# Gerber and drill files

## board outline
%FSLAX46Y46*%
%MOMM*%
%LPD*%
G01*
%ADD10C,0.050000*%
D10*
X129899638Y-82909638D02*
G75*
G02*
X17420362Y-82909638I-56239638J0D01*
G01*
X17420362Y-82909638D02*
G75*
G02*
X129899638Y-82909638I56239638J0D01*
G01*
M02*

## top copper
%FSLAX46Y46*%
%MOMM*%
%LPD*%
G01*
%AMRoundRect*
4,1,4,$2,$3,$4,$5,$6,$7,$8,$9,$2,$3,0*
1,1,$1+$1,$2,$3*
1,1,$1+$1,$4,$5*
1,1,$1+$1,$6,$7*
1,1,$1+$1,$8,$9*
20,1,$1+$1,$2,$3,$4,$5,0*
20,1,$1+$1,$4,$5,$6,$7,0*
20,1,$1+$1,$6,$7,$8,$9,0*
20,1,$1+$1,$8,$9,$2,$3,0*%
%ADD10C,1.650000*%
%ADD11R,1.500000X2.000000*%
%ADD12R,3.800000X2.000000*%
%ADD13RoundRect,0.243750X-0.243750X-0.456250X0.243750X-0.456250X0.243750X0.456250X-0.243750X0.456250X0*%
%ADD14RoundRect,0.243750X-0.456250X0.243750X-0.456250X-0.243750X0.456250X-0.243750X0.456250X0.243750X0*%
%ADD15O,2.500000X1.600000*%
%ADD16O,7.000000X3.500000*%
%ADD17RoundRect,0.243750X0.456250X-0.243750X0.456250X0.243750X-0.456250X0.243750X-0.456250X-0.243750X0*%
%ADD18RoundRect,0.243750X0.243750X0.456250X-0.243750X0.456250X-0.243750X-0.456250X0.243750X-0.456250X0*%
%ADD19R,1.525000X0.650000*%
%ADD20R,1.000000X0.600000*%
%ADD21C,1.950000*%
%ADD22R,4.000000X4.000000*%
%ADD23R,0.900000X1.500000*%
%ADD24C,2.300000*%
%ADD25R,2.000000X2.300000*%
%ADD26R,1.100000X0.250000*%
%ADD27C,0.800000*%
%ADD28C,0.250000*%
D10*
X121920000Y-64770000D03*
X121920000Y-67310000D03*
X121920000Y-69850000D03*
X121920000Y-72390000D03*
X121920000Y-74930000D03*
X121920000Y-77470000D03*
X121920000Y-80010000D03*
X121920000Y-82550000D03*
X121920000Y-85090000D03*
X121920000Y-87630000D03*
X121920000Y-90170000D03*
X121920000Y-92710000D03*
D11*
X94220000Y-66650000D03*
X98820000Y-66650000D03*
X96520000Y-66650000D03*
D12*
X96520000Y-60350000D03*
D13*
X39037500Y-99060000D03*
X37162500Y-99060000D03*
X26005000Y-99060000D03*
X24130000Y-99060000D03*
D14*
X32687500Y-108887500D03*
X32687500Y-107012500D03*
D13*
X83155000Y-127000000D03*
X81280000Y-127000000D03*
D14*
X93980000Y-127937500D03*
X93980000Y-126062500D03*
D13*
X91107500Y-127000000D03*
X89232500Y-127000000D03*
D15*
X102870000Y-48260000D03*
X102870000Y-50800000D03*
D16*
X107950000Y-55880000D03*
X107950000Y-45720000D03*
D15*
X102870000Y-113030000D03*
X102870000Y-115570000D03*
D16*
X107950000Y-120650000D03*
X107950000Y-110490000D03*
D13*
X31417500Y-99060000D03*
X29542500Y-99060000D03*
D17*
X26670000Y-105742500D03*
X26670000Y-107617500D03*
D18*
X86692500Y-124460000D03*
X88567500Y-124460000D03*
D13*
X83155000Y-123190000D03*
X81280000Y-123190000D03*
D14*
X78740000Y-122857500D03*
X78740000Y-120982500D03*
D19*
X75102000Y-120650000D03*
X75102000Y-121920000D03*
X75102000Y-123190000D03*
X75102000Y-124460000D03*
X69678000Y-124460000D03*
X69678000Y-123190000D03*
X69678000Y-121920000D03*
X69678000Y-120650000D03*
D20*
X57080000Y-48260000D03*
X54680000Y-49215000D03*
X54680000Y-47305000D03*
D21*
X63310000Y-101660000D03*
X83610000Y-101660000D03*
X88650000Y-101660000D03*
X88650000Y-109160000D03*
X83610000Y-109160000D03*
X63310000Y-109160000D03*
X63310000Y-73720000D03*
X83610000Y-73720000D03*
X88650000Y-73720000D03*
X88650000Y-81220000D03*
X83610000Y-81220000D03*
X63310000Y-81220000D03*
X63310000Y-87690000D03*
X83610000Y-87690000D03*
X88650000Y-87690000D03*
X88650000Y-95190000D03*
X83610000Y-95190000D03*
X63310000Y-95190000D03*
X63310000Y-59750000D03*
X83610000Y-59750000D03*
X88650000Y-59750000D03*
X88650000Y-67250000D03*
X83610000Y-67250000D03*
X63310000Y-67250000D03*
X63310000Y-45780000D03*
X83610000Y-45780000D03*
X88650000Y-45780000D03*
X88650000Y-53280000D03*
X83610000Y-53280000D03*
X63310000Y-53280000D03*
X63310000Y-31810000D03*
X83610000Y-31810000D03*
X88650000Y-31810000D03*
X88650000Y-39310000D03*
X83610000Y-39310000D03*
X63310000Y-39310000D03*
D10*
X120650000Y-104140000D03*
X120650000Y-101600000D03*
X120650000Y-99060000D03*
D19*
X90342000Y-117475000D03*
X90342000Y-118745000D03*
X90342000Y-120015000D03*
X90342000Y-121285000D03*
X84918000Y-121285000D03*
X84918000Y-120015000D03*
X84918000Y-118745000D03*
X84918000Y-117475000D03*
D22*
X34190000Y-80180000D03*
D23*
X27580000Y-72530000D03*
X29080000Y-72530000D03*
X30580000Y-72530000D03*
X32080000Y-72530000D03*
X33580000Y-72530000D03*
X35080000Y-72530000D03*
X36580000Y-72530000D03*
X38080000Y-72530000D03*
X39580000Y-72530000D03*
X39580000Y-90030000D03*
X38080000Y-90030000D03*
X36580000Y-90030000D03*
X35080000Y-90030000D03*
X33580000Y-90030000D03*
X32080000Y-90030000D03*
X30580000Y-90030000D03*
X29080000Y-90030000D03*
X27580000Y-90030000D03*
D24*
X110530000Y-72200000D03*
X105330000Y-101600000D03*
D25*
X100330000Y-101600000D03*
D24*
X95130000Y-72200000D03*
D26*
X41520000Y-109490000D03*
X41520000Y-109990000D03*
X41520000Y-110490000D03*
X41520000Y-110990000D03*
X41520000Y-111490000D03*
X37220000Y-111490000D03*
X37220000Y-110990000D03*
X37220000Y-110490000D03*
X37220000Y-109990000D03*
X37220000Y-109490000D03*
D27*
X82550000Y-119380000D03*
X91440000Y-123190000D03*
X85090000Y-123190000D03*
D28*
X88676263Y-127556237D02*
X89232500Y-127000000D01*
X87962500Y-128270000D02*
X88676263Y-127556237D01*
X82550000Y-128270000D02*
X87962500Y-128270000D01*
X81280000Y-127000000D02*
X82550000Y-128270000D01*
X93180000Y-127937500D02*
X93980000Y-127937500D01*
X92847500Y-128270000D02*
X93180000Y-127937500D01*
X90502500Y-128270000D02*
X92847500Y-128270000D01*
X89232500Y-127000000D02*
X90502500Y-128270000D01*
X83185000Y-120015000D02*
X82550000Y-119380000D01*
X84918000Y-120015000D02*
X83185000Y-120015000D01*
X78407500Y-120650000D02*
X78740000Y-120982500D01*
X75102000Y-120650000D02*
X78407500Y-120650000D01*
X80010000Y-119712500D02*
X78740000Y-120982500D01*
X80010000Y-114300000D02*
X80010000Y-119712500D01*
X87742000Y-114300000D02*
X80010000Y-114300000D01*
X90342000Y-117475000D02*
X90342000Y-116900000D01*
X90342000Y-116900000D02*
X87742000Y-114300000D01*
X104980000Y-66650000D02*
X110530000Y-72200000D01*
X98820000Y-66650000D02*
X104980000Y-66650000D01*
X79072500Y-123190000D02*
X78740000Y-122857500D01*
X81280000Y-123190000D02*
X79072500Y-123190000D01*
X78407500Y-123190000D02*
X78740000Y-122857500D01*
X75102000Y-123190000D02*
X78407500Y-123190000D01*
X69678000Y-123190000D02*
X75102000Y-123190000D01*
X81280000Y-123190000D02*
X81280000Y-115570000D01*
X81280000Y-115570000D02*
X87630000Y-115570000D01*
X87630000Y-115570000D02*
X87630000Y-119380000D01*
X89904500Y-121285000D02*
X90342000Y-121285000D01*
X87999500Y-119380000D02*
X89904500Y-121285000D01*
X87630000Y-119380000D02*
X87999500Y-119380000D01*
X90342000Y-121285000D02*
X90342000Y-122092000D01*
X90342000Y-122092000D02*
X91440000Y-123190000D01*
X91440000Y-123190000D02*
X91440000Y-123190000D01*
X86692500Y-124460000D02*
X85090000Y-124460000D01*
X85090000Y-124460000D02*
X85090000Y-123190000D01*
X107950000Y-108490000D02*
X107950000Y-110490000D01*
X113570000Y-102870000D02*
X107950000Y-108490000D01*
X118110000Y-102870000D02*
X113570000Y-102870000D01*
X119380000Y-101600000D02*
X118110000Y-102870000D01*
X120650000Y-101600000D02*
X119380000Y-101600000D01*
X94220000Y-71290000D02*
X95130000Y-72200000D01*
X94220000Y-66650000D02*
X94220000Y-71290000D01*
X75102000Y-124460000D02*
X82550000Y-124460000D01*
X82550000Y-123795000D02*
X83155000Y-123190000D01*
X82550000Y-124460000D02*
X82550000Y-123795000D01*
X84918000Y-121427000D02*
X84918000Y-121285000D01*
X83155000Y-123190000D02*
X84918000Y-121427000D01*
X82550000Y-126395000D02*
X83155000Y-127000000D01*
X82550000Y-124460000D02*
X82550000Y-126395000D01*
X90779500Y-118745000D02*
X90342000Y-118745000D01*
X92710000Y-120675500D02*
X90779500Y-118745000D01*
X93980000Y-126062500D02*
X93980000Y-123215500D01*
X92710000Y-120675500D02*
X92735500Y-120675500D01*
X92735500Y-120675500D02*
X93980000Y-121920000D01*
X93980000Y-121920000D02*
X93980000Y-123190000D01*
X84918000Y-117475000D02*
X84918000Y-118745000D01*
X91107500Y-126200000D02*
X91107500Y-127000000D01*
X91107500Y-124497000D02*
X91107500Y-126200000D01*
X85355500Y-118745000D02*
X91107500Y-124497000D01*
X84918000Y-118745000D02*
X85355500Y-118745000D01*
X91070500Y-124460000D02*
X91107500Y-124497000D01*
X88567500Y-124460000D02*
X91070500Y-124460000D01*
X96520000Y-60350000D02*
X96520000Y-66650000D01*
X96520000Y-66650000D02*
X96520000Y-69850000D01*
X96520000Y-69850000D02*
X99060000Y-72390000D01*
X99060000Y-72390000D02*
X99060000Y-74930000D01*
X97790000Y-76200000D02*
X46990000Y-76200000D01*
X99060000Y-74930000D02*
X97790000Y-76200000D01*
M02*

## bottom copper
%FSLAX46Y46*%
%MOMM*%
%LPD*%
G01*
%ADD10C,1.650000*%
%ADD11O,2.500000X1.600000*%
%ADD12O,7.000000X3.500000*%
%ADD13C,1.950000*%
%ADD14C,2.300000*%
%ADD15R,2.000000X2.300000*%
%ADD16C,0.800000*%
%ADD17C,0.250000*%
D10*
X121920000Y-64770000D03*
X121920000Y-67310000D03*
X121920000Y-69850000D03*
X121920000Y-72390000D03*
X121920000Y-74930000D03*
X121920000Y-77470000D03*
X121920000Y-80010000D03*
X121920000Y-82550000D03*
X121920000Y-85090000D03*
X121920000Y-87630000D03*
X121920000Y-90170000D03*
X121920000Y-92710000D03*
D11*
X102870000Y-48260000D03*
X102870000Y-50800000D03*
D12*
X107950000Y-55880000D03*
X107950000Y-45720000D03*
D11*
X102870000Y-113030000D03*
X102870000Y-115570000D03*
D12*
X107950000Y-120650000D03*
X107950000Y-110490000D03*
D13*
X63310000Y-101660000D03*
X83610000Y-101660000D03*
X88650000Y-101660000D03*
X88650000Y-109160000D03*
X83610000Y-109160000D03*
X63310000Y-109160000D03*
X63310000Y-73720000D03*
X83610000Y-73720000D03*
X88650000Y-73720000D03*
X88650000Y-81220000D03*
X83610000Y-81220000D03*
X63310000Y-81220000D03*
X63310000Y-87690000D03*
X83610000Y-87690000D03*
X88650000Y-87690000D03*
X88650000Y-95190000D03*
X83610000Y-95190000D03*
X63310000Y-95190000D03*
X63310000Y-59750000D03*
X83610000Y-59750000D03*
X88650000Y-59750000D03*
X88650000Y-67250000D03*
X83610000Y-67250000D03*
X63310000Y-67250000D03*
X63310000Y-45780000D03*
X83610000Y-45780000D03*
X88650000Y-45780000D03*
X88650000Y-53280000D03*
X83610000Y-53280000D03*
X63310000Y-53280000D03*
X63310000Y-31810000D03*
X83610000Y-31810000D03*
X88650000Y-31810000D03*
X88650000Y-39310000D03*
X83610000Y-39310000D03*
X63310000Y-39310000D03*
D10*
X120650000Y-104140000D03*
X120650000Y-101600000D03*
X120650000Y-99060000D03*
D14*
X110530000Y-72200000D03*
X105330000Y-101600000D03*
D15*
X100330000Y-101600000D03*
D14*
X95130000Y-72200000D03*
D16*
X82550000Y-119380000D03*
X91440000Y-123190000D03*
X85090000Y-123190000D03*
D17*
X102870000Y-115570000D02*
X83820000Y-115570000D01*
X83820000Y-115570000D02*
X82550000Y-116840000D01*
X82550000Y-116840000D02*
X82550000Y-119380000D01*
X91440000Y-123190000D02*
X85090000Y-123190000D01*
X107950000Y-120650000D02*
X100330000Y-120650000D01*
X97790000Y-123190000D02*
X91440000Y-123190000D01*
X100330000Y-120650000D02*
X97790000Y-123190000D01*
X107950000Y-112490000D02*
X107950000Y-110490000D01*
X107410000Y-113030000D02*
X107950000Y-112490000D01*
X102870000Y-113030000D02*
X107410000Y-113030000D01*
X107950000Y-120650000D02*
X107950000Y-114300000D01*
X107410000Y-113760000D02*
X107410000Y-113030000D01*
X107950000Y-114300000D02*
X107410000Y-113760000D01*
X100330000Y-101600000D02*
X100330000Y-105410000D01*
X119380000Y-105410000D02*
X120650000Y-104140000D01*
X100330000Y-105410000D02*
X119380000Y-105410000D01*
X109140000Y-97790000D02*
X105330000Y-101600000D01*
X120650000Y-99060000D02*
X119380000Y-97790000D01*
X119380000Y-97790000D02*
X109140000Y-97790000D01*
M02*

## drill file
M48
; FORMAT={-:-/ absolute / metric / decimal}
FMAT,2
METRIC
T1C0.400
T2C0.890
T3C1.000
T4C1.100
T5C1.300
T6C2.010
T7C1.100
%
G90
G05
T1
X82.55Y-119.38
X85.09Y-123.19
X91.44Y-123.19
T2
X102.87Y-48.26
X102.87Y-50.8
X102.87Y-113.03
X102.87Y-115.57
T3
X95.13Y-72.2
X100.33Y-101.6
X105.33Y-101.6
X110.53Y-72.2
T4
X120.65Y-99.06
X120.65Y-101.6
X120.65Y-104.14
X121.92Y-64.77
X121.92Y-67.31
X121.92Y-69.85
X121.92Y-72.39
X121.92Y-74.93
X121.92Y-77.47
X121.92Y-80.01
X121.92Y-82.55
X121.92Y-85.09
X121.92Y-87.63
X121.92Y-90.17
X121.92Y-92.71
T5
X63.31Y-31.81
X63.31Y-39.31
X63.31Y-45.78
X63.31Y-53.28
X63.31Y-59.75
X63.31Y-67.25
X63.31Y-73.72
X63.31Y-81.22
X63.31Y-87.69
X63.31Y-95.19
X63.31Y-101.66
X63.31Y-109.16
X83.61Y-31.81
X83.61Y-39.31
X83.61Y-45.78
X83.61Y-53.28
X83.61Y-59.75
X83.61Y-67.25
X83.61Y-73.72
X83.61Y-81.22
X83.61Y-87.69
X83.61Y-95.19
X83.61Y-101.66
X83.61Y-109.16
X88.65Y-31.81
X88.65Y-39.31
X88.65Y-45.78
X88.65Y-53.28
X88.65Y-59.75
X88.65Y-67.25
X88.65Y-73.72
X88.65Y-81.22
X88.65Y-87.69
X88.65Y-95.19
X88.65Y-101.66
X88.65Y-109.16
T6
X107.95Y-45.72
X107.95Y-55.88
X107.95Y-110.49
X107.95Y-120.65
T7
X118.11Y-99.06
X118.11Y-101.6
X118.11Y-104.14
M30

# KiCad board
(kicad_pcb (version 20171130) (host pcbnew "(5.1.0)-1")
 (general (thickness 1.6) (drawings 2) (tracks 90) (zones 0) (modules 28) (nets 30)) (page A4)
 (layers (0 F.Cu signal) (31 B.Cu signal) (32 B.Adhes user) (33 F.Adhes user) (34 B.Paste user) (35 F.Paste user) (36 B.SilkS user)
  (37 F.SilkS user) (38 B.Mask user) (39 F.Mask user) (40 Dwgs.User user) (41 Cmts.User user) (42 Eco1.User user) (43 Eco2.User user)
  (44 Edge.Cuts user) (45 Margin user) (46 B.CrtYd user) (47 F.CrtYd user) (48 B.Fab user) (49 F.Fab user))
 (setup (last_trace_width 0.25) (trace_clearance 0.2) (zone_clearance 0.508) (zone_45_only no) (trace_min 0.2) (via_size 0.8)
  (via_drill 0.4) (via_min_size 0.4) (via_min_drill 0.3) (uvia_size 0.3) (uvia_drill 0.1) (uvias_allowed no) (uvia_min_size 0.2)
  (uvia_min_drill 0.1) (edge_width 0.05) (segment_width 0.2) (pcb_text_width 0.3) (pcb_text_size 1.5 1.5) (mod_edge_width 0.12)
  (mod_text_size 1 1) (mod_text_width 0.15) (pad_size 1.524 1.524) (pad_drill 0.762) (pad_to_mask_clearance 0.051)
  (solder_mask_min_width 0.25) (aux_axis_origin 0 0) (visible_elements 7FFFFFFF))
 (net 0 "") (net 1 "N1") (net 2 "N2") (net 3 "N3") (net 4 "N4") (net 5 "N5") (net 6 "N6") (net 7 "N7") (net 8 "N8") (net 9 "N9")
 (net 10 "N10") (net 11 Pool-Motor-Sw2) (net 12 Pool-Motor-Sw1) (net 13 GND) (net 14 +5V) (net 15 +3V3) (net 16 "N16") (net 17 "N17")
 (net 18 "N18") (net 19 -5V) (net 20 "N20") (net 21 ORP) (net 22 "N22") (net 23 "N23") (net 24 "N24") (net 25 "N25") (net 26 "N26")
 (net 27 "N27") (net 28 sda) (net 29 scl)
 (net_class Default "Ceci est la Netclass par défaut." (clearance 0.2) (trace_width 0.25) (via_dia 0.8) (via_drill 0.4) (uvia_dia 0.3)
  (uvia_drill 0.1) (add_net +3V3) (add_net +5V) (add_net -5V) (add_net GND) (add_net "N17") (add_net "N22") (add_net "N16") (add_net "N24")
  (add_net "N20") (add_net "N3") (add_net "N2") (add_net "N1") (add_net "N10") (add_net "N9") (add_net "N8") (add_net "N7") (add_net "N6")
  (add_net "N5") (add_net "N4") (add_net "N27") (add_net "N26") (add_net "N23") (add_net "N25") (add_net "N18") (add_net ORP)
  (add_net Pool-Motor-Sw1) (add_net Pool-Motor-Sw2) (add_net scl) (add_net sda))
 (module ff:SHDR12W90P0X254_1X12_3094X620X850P (layer F.Cu) (at 121.92 92.71 90)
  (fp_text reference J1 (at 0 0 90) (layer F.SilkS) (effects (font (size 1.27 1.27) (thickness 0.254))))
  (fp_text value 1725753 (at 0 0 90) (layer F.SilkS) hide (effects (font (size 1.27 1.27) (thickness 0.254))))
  (pad 12 thru_hole circle (at 27.94 0 90) (size 1.65 1.65) (drill 1.1) (layers *.Cu *.Mask) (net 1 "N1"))
  (pad 11 thru_hole circle (at 25.4 0 90) (size 1.65 1.65) (drill 1.1) (layers *.Cu *.Mask) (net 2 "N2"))
  (pad 10 thru_hole circle (at 22.86 0 90) (size 1.65 1.65) (drill 1.1) (layers *.Cu *.Mask) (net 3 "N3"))
  (pad 9 thru_hole circle (at 20.32 0 90) (size 1.65 1.65) (drill 1.1) (layers *.Cu *.Mask) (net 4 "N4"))
  (pad 8 thru_hole circle (at 17.78 0 90) (size 1.65 1.65) (drill 1.1) (layers *.Cu *.Mask) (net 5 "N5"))
  (pad 7 thru_hole circle (at 15.24 0 90) (size 1.65 1.65) (drill 1.1) (layers *.Cu *.Mask) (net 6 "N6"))
  (pad 6 thru_hole circle (at 12.7 0 90) (size 1.65 1.65) (drill 1.1) (layers *.Cu *.Mask) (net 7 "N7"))
  (pad 5 thru_hole circle (at 10.16 0 90) (size 1.65 1.65) (drill 1.1) (layers *.Cu *.Mask) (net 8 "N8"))
  (pad 4 thru_hole circle (at 7.62 0 90) (size 1.65 1.65) (drill 1.1) (layers *.Cu *.Mask) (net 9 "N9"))
  (pad 3 thru_hole circle (at 5.08 0 90) (size 1.65 1.65) (drill 1.1) (layers *.Cu *.Mask) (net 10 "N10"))
  (pad 2 thru_hole circle (at 2.54 0 90) (size 1.65 1.65) (drill 1.1) (layers *.Cu *.Mask) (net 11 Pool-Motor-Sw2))
  (pad 1 thru_hole circle (at 0 0 90) (size 1.65 1.65) (drill 1.1) (layers *.Cu *.Mask) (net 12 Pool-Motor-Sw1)))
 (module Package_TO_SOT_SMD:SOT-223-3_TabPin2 (layer F.Cu) (at 96.52 63.5 90)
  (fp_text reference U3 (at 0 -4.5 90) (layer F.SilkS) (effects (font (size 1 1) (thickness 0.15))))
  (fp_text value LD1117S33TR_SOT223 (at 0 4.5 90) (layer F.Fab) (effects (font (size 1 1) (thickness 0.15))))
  (pad 1 smd rect (at -3.15 -2.3 90) (size 2 1.5) (layers F.Cu F.Paste F.Mask) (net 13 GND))
  (pad 3 smd rect (at -3.15 2.3 90) (size 2 1.5) (layers F.Cu F.Paste F.Mask) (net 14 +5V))
  (pad 2 smd rect (at -3.15 0 90) (size 2 1.5) (layers F.Cu F.Paste F.Mask) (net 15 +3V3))
  (pad 2 smd rect (at 3.15 0 90) (size 2 3.8) (layers F.Cu F.Paste F.Mask) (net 15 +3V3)))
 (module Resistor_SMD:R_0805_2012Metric (layer F.Cu) (at 38.1 99.06)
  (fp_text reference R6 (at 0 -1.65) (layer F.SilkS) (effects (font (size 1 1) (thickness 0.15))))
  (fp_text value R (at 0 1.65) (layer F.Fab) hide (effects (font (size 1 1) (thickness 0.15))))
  (pad 2 smd roundrect (at 0.9375 0) (size 0.975 1.4) (layers F.Cu F.Paste F.Mask) (roundrect_rratio 0.25) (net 13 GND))
  (pad 1 smd roundrect (at -0.9375 0) (size 0.975 1.4) (layers F.Cu F.Paste F.Mask) (roundrect_rratio 0.25) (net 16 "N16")))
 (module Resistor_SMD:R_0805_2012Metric (layer F.Cu) (at 25.0675 99.06)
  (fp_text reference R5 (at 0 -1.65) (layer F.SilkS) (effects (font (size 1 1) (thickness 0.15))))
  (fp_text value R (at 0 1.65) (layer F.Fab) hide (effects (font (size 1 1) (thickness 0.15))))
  (pad 2 smd roundrect (at 0.9375 0) (size 0.975 1.4) (layers F.Cu F.Paste F.Mask) (roundrect_rratio 0.25) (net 15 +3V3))
  (pad 1 smd roundrect (at -0.9375 0) (size 0.975 1.4) (layers F.Cu F.Paste F.Mask) (roundrect_rratio 0.25) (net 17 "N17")))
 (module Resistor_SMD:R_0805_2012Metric (layer F.Cu) (at 32.6875 107.95 270)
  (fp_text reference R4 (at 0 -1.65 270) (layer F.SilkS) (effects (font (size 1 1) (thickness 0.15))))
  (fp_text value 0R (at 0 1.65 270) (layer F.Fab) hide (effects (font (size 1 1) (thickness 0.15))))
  (pad 2 smd roundrect (at 0.9375 0 270) (size 0.975 1.4) (layers F.Cu F.Paste F.Mask) (roundrect_rratio 0.25) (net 13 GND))
  (pad 1 smd roundrect (at -0.9375 0 270) (size 0.975 1.4) (layers F.Cu F.Paste F.Mask) (roundrect_rratio 0.25) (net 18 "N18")))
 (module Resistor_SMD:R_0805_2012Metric (layer F.Cu) (at 82.2175 127)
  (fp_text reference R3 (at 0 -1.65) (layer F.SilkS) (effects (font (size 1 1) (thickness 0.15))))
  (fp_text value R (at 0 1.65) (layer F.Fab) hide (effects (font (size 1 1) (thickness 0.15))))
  (pad 2 smd roundrect (at 0.9375 0) (size 0.975 1.4) (layers F.Cu F.Paste F.Mask) (roundrect_rratio 0.25) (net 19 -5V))
  (pad 1 smd roundrect (at -0.9375 0) (size 0.975 1.4) (layers F.Cu F.Paste F.Mask) (roundrect_rratio 0.25) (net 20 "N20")))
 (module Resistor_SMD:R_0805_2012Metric (layer F.Cu) (at 93.98 127 270)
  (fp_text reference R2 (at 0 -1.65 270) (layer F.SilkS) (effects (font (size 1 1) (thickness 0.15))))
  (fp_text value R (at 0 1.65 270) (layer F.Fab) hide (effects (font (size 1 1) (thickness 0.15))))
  (pad 2 smd roundrect (at 0.9375 0 270) (size 0.975 1.4) (layers F.Cu F.Paste F.Mask) (roundrect_rratio 0.25) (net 20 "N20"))
  (pad 1 smd roundrect (at -0.9375 0 270) (size 0.975 1.4) (layers F.Cu F.Paste F.Mask) (roundrect_rratio 0.25) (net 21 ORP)))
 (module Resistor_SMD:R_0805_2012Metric (layer F.Cu) (at 90.17 127)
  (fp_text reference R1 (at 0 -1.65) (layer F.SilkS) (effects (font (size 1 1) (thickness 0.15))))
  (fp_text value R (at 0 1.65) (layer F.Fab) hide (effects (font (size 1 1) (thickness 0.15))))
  (pad 2 smd roundrect (at 0.9375 0) (size 0.975 1.4) (layers F.Cu F.Paste F.Mask) (roundrect_rratio 0.25) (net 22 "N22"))
  (pad 1 smd roundrect (at -0.9375 0) (size 0.975 1.4) (layers F.Cu F.Paste F.Mask) (roundrect_rratio 0.25) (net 20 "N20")))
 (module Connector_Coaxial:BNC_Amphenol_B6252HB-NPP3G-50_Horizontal (layer F.Cu) (at 102.87 50.8 270)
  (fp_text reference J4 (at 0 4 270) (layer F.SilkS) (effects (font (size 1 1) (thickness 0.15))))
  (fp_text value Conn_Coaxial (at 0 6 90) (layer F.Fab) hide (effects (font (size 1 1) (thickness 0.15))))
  (pad 2 thru_hole oval (at -2.54 0 270) (size 1.6 2.5) (drill 0.89) (layers *.Cu *.Mask) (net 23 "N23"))
  (pad 1 thru_hole oval (at 0 0 270) (size 1.6 2.5) (drill 0.89) (layers *.Cu *.Mask))
  (pad 2 thru_hole oval (at 5.08 -5.08 270) (size 3.5 7) (drill 2.01) (layers *.Cu *.Mask) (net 23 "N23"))
  (pad 2 thru_hole oval (at -5.08 -5.08 270) (size 3.5 7) (drill 2.01) (layers *.Cu *.Mask) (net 23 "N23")))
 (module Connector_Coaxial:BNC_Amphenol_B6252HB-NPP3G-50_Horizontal (layer F.Cu) (at 102.87 115.57 270)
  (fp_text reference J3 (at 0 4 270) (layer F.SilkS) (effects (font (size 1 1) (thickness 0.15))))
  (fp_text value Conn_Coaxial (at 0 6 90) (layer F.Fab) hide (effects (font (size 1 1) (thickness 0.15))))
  (pad 2 thru_hole oval (at -2.54 0 270) (size 1.6 2.5) (drill 0.89) (layers *.Cu *.Mask) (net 13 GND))
  (pad 1 thru_hole oval (at 0 0 270) (size 1.6 2.5) (drill 0.89) (layers *.Cu *.Mask) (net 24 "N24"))
  (pad 2 thru_hole oval (at 5.08 -5.08 270) (size 3.5 7) (drill 2.01) (layers *.Cu *.Mask) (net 13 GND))
  (pad 2 thru_hole oval (at -5.08 -5.08 270) (size 3.5 7) (drill 2.01) (layers *.Cu *.Mask) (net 13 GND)))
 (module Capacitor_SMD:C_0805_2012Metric (layer F.Cu) (at 30.48 99.06)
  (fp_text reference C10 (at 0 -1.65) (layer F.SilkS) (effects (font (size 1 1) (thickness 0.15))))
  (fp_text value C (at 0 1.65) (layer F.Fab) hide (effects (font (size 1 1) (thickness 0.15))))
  (pad 2 smd roundrect (at 0.9375 0) (size 0.975 1.4) (layers F.Cu F.Paste F.Mask) (roundrect_rratio 0.25) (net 13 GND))
  (pad 1 smd roundrect (at -0.9375 0) (size 0.975 1.4) (layers F.Cu F.Paste F.Mask) (roundrect_rratio 0.25) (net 17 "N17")))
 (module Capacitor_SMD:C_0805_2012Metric (layer F.Cu) (at 26.67 106.68 90)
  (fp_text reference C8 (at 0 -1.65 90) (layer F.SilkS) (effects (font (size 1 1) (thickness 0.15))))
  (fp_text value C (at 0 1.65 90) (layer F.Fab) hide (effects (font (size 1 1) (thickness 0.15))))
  (pad 2 smd roundrect (at 0.9375 0 90) (size 0.975 1.4) (layers F.Cu F.Paste F.Mask) (roundrect_rratio 0.25) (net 13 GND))
  (pad 1 smd roundrect (at -0.9375 0 90) (size 0.975 1.4) (layers F.Cu F.Paste F.Mask) (roundrect_rratio 0.25) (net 15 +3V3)))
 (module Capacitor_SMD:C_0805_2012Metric (layer F.Cu) (at 87.63 124.46 180)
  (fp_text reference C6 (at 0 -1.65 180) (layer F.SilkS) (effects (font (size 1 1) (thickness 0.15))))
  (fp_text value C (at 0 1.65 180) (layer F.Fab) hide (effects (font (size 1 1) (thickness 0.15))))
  (pad 2 smd roundrect (at 0.9375 0 180) (size 0.975 1.4) (layers F.Cu F.Paste F.Mask) (roundrect_rratio 0.25) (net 13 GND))
  (pad 1 smd roundrect (at -0.9375 0 180) (size 0.975 1.4) (layers F.Cu F.Paste F.Mask) (roundrect_rratio 0.25) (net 22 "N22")))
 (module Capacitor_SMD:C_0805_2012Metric (layer F.Cu) (at 82.2175 123.19)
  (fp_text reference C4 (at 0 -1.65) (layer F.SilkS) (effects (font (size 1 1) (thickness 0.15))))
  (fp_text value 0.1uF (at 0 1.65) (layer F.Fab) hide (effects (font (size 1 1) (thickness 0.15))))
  (pad 2 smd roundrect (at 0.9375 0) (size 0.975 1.4) (layers F.Cu F.Paste F.Mask) (roundrect_rratio 0.25) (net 19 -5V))
  (pad 1 smd roundrect (at -0.9375 0) (size 0.975 1.4) (layers F.Cu F.Paste F.Mask) (roundrect_rratio 0.25) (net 13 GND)))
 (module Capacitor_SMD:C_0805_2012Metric (layer F.Cu) (at 78.74 121.92 270)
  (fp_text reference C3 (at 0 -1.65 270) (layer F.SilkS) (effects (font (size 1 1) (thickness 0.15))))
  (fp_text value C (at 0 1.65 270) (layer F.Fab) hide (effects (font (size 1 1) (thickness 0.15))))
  (pad 2 smd roundrect (at 0.9375 0 270) (size 0.975 1.4) (layers F.Cu F.Paste F.Mask) (roundrect_rratio 0.25) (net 13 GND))
  (pad 1 smd roundrect (at -0.9375 0 270) (size 0.975 1.4) (layers F.Cu F.Paste F.Mask) (roundrect_rratio 0.25) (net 14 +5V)))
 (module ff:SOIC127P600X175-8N (layer F.Cu) (at 72.39 122.555)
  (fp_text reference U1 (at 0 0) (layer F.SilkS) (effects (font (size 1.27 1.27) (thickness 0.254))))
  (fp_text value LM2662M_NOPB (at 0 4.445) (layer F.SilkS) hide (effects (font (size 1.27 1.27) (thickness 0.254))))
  (pad 8 smd rect (at 2.712 -1.905 90) (size 0.65 1.525) (layers F.Cu F.Paste F.Mask) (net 14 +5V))
  (pad 7 smd rect (at 2.712 -0.635 90) (size 0.65 1.525) (layers F.Cu F.Paste F.Mask))
  (pad 6 smd rect (at 2.712 0.635 90) (size 0.65 1.525) (layers F.Cu F.Paste F.Mask) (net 13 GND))
  (pad 5 smd rect (at 2.712 1.905 90) (size 0.65 1.525) (layers F.Cu F.Paste F.Mask) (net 19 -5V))
  (pad 4 smd rect (at -2.712 1.905 90) (size 0.65 1.525) (layers F.Cu F.Paste F.Mask))
  (pad 3 smd rect (at -2.712 0.635 90) (size 0.65 1.525) (layers F.Cu F.Paste F.Mask) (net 13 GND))
  (pad 2 smd rect (at -2.712 -0.635 90) (size 0.65 1.525) (layers F.Cu F.Paste F.Mask))
  (pad 1 smd rect (at -2.712 -1.905 90) (size 0.65 1.525) (layers F.Cu F.Paste F.Mask)))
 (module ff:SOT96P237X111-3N (layer F.Cu) (at 55.88 48.26)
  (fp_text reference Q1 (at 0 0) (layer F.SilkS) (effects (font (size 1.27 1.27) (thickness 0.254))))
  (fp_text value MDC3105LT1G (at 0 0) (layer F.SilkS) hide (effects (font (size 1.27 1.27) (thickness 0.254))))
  (pad 3 smd rect (at 1.2 0 90) (size 0.6 1) (layers F.Cu F.Paste F.Mask) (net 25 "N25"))
  (pad 2 smd rect (at -1.2 0.955 90) (size 0.6 1) (layers F.Cu F.Paste F.Mask) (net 13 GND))
  (pad 1 smd rect (at -1.2 -0.955 90) (size 0.6 1) (layers F.Cu F.Paste F.Mask)))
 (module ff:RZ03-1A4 (layer F.Cu) (at 60.96 111.76)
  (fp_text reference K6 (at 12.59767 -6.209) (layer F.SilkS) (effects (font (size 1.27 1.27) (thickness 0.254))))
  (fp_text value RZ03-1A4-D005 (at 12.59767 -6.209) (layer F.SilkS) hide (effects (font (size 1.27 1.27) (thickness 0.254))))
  (pad 6 thru_hole circle (at 2.35 -10.1) (size 1.95 1.95) (drill 1.3) (layers *.Cu *.Mask))
  (pad 5 thru_hole circle (at 22.65 -10.1) (size 1.95 1.95) (drill 1.3) (layers *.Cu *.Mask))
  (pad 4 thru_hole circle (at 27.69 -10.1) (size 1.95 1.95) (drill 1.3) (layers *.Cu *.Mask))
  (pad 3 thru_hole circle (at 27.69 -2.6) (size 1.95 1.95) (drill 1.3) (layers *.Cu *.Mask))
  (pad 2 thru_hole circle (at 22.65 -2.6) (size 1.95 1.95) (drill 1.3) (layers *.Cu *.Mask))
  (pad 1 thru_hole circle (at 2.35 -2.6) (size 1.95 1.95) (drill 1.3) (layers *.Cu *.Mask)))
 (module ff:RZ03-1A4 (layer F.Cu) (at 60.96 83.82)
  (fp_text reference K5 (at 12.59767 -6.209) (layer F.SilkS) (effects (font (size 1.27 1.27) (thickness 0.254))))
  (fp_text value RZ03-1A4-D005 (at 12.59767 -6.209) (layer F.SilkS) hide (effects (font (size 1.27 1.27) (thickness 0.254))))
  (pad 6 thru_hole circle (at 2.35 -10.1) (size 1.95 1.95) (drill 1.3) (layers *.Cu *.Mask))
  (pad 5 thru_hole circle (at 22.65 -10.1) (size 1.95 1.95) (drill 1.3) (layers *.Cu *.Mask))
  (pad 4 thru_hole circle (at 27.69 -10.1) (size 1.95 1.95) (drill 1.3) (layers *.Cu *.Mask))
  (pad 3 thru_hole circle (at 27.69 -2.6) (size 1.95 1.95) (drill 1.3) (layers *.Cu *.Mask))
  (pad 2 thru_hole circle (at 22.65 -2.6) (size 1.95 1.95) (drill 1.3) (layers *.Cu *.Mask))
  (pad 1 thru_hole circle (at 2.35 -2.6) (size 1.95 1.95) (drill 1.3) (layers *.Cu *.Mask)))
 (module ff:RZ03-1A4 (layer F.Cu) (at 60.96 97.79)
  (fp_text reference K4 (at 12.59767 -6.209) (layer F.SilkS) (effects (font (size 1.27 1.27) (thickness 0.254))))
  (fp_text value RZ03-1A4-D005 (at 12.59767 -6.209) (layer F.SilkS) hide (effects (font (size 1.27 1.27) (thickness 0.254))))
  (pad 6 thru_hole circle (at 2.35 -10.1) (size 1.95 1.95) (drill 1.3) (layers *.Cu *.Mask))
  (pad 5 thru_hole circle (at 22.65 -10.1) (size 1.95 1.95) (drill 1.3) (layers *.Cu *.Mask))
  (pad 4 thru_hole circle (at 27.69 -10.1) (size 1.95 1.95) (drill 1.3) (layers *.Cu *.Mask))
  (pad 3 thru_hole circle (at 27.69 -2.6) (size 1.95 1.95) (drill 1.3) (layers *.Cu *.Mask))
  (pad 2 thru_hole circle (at 22.65 -2.6) (size 1.95 1.95) (drill 1.3) (layers *.Cu *.Mask))
  (pad 1 thru_hole circle (at 2.35 -2.6) (size 1.95 1.95) (drill 1.3) (layers *.Cu *.Mask)))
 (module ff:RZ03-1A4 (layer F.Cu) (at 60.96 69.85)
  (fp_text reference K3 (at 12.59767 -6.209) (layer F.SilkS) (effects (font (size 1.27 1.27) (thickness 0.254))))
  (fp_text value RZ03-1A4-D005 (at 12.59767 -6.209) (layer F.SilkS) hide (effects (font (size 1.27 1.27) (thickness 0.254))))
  (pad 6 thru_hole circle (at 2.35 -10.1) (size 1.95 1.95) (drill 1.3) (layers *.Cu *.Mask))
  (pad 5 thru_hole circle (at 22.65 -10.1) (size 1.95 1.95) (drill 1.3) (layers *.Cu *.Mask))
  (pad 4 thru_hole circle (at 27.69 -10.1) (size 1.95 1.95) (drill 1.3) (layers *.Cu *.Mask))
  (pad 3 thru_hole circle (at 27.69 -2.6) (size 1.95 1.95) (drill 1.3) (layers *.Cu *.Mask))
  (pad 2 thru_hole circle (at 22.65 -2.6) (size 1.95 1.95) (drill 1.3) (layers *.Cu *.Mask))
  (pad 1 thru_hole circle (at 2.35 -2.6) (size 1.95 1.95) (drill 1.3) (layers *.Cu *.Mask)))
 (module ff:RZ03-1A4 (layer F.Cu) (at 60.96 55.88)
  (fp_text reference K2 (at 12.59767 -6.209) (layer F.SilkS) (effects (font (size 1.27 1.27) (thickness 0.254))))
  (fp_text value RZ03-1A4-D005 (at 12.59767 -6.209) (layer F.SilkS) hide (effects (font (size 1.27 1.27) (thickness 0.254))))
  (pad 6 thru_hole circle (at 2.35 -10.1) (size 1.95 1.95) (drill 1.3) (layers *.Cu *.Mask))
  (pad 5 thru_hole circle (at 22.65 -10.1) (size 1.95 1.95) (drill 1.3) (layers *.Cu *.Mask))
  (pad 4 thru_hole circle (at 27.69 -10.1) (size 1.95 1.95) (drill 1.3) (layers *.Cu *.Mask))
  (pad 3 thru_hole circle (at 27.69 -2.6) (size 1.95 1.95) (drill 1.3) (layers *.Cu *.Mask))
  (pad 2 thru_hole circle (at 22.65 -2.6) (size 1.95 1.95) (drill 1.3) (layers *.Cu *.Mask))
  (pad 1 thru_hole circle (at 2.35 -2.6) (size 1.95 1.95) (drill 1.3) (layers *.Cu *.Mask)))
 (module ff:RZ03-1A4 (layer F.Cu) (at 60.96 41.91)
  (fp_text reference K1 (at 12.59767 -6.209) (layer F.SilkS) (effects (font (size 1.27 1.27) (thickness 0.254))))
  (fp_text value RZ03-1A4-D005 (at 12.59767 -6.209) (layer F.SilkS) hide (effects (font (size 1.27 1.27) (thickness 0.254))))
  (pad 6 thru_hole circle (at 2.35 -10.1) (size 1.95 1.95) (drill 1.3) (layers *.Cu *.Mask) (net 14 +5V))
  (pad 5 thru_hole circle (at 22.65 -10.1) (size 1.95 1.95) (drill 1.3) (layers *.Cu *.Mask))
  (pad 4 thru_hole circle (at 27.69 -10.1) (size 1.95 1.95) (drill 1.3) (layers *.Cu *.Mask))
  (pad 3 thru_hole circle (at 27.69 -2.6) (size 1.95 1.95) (drill 1.3) (layers *.Cu *.Mask))
  (pad 2 thru_hole circle (at 22.65 -2.6) (size 1.95 1.95) (drill 1.3) (layers *.Cu *.Mask))
  (pad 1 thru_hole circle (at 2.35 -2.6) (size 1.95 1.95) (drill 1.3) (layers *.Cu *.Mask) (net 25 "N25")))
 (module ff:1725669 (layer F.Cu) (at 120.65 99.06 270)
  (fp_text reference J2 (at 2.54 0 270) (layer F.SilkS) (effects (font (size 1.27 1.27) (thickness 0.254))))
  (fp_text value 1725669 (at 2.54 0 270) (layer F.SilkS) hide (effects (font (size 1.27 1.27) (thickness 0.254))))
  (pad 6 np_thru_hole circle (at 5.08 2.54 270) (size 1.1 0) (drill 1.1) (layers *.Cu *.Mask))
  (pad 5 np_thru_hole circle (at 2.54 2.54 270) (size 1.1 0) (drill 1.1) (layers *.Cu *.Mask))
  (pad 4 np_thru_hole circle (at 0 2.54 270) (size 1.1 0) (drill 1.1) (layers *.Cu *.Mask))
  (pad 3 thru_hole circle (at 5.08 0 270) (size 1.65 1.65) (drill 1.1) (layers *.Cu *.Mask) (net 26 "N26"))
  (pad 2 thru_hole circle (at 2.54 0 270) (size 1.65 1.65) (drill 1.1) (layers *.Cu *.Mask) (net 13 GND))
  (pad 1 thru_hole circle (at 0 0 270) (size 1.65 1.65) (drill 1.1) (layers *.Cu *.Mask) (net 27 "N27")))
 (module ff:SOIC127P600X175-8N (layer F.Cu) (at 87.63 119.38)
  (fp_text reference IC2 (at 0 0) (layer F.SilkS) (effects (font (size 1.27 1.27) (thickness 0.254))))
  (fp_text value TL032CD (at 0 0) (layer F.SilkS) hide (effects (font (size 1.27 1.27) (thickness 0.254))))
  (pad 8 smd rect (at 2.712 -1.905 90) (size 0.65 1.525) (layers F.Cu F.Paste F.Mask) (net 14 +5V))
  (pad 7 smd rect (at 2.712 -0.635 90) (size 0.65 1.525) (layers F.Cu F.Paste F.Mask) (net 21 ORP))
  (pad 6 smd rect (at 2.712 0.635 90) (size 0.65 1.525) (layers F.Cu F.Paste F.Mask) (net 20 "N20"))
  (pad 5 smd rect (at 2.712 1.905 90) (size 0.65 1.525) (layers F.Cu F.Paste F.Mask) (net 13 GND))
  (pad 4 smd rect (at -2.712 1.905 90) (size 0.65 1.525) (layers F.Cu F.Paste F.Mask) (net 19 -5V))
  (pad 3 smd rect (at -2.712 0.635 90) (size 0.65 1.525) (layers F.Cu F.Paste F.Mask) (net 24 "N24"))
  (pad 2 smd rect (at -2.712 -0.635 90) (size 0.65 1.525) (layers F.Cu F.Paste F.Mask) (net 22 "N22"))
  (pad 1 smd rect (at -2.712 -1.905 90) (size 0.65 1.525) (layers F.Cu F.Paste F.Mask) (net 22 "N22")))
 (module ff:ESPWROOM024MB (layer F.Cu) (at 30.48 81.28 90)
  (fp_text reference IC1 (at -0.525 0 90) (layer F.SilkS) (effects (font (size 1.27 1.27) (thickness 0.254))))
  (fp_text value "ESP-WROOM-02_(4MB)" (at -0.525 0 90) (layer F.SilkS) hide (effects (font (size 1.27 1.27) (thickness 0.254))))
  (pad 19 smd rect (at 1.1 3.71 180) (size 4 4) (layers F.Cu F.Paste F.Mask) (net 13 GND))
  (pad 18 smd rect (at 8.75 -2.9 180) (size 0.9 1.5) (layers F.Cu F.Paste F.Mask) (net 13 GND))
  (pad 17 smd rect (at 8.75 -1.4 180) (size 0.9 1.5) (layers F.Cu F.Paste F.Mask))
  (pad 16 smd rect (at 8.75 0.1 180) (size 0.9 1.5) (layers F.Cu F.Paste F.Mask))
  (pad 15 smd rect (at 8.75 1.6 180) (size 0.9 1.5) (layers F.Cu F.Paste F.Mask))
  (pad 14 smd rect (at 8.75 3.1 180) (size 0.9 1.5) (layers F.Cu F.Paste F.Mask))
  (pad 13 smd rect (at 8.75 4.6 180) (size 0.9 1.5) (layers F.Cu F.Paste F.Mask))
  (pad 12 smd rect (at 8.75 6.1 180) (size 0.9 1.5) (layers F.Cu F.Paste F.Mask))
  (pad 11 smd rect (at 8.75 7.6 180) (size 0.9 1.5) (layers F.Cu F.Paste F.Mask))
  (pad 10 smd rect (at 8.75 9.1 180) (size 0.9 1.5) (layers F.Cu F.Paste F.Mask))
  (pad 9 smd rect (at -8.75 9.1 180) (size 0.9 1.5) (layers F.Cu F.Paste F.Mask) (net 13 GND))
  (pad 8 smd rect (at -8.75 7.6 180) (size 0.9 1.5) (layers F.Cu F.Paste F.Mask))
  (pad 7 smd rect (at -8.75 6.1 180) (size 0.9 1.5) (layers F.Cu F.Paste F.Mask) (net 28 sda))
  (pad 6 smd rect (at -8.75 4.6 180) (size 0.9 1.5) (layers F.Cu F.Paste F.Mask) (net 16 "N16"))
  (pad 5 smd rect (at -8.75 3.1 180) (size 0.9 1.5) (layers F.Cu F.Paste F.Mask))
  (pad 4 smd rect (at -8.75 1.6 180) (size 0.9 1.5) (layers F.Cu F.Paste F.Mask))
  (pad 3 smd rect (at -8.75 0.1 180) (size 0.9 1.5) (layers F.Cu F.Paste F.Mask) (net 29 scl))
  (pad 2 smd rect (at -8.75 -1.4 180) (size 0.9 1.5) (layers F.Cu F.Paste F.Mask) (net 17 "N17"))
  (pad 1 smd rect (at -8.75 -2.9 180) (size 0.9 1.5) (layers F.Cu F.Paste F.Mask)))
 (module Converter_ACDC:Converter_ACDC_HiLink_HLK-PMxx (layer F.Cu) (at 100.33 101.6 90)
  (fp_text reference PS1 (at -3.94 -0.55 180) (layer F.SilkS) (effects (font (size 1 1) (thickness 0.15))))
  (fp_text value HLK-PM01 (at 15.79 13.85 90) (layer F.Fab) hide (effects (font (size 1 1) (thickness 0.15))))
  (pad 4 thru_hole circle (at 29.4 10.2 90) (size 2.3 2.3) (drill 1) (layers *.Cu *.Mask) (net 14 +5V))
  (pad 2 thru_hole circle (at 0 5 90) (size 2.3 2.3) (drill 1) (layers *.Cu *.Mask) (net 27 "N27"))
  (pad 1 thru_hole rect (at 0 0 90) (size 2.3 2) (drill 1) (layers *.Cu *.Mask) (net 26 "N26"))
  (pad 3 thru_hole circle (at 29.4 -5.2 90) (size 2.3 2.3) (drill 1) (layers *.Cu *.Mask) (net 13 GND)))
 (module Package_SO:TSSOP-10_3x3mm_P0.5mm (layer F.Cu) (at 39.37 110.49)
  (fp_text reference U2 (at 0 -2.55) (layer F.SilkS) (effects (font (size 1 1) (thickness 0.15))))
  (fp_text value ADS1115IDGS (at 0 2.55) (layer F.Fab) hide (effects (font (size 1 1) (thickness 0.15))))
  (pad 10 smd rect (at 2.15 -1) (size 1.1 0.25) (layers F.Cu F.Paste F.Mask) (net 29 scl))
  (pad 9 smd rect (at 2.15 -0.5) (size 1.1 0.25) (layers F.Cu F.Paste F.Mask) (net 28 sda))
  (pad 8 smd rect (at 2.15 0) (size 1.1 0.25) (layers F.Cu F.Paste F.Mask) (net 14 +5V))
  (pad 7 smd rect (at 2.15 0.5) (size 1.1 0.25) (layers F.Cu F.Paste F.Mask))
  (pad 6 smd rect (at 2.15 1) (size 1.1 0.25) (layers F.Cu F.Paste F.Mask))
  (pad 5 smd rect (at -2.15 1) (size 1.1 0.25) (layers F.Cu F.Paste F.Mask))
  (pad 4 smd rect (at -2.15 0.5) (size 1.1 0.25) (layers F.Cu F.Paste F.Mask) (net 21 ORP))
  (pad 3 smd rect (at -2.15 0) (size 1.1 0.25) (layers F.Cu F.Paste F.Mask) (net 13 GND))
  (pad 2 smd rect (at -2.15 -0.5) (size 1.1 0.25) (layers F.Cu F.Paste F.Mask))
  (pad 1 smd rect (at -2.15 -1) (size 1.1 0.25) (layers F.Cu F.Paste F.Mask) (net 18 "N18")))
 (gr_circle (center 73.66 82.909638) (end 129.54 89.259638) (layer Edge.Cuts) (width 0.05))
 (segment (start 88.676263 127.556237) (end 89.2325 127) (width 0.25) (layer F.Cu) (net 20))
 (segment (start 87.9625 128.27) (end 88.676263 127.556237) (width 0.25) (layer F.Cu) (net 20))
 (segment (start 82.55 128.27) (end 87.9625 128.27) (width 0.25) (layer F.Cu) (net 20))
 (segment (start 81.28 127) (end 82.55 128.27) (width 0.25) (layer F.Cu) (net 20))
 (segment (start 93.18 127.9375) (end 93.98 127.9375) (width 0.25) (layer F.Cu) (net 20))
 (segment (start 92.8475 128.27) (end 93.18 127.9375) (width 0.25) (layer F.Cu) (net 20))
 (segment (start 90.5025 128.27) (end 92.8475 128.27) (width 0.25) (layer F.Cu) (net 20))
 (segment (start 89.2325 127) (end 90.5025 128.27) (width 0.25) (layer F.Cu) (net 20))
 (segment (start 102.87 115.57) (end 83.82 115.57) (width 0.25) (layer B.Cu) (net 24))
 (segment (start 83.82 115.57) (end 82.55 116.84) (width 0.25) (layer B.Cu) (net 24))
 (via (at 82.55 119.38) (size 0.8) (drill 0.4) (layers F.Cu B.Cu) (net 24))
 (segment (start 82.55 116.84) (end 82.55 119.38) (width 0.25) (layer B.Cu) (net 24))
 (segment (start 83.185 120.015) (end 82.55 119.38) (width 0.25) (layer F.Cu) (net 24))
 (segment (start 84.918 120.015) (end 83.185 120.015) (width 0.25) (layer F.Cu) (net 24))
 (segment (start 78.4075 120.65) (end 78.74 120.9825) (width 0.25) (layer F.Cu) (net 14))
 (segment (start 75.102 120.65) (end 78.4075 120.65) (width 0.25) (layer F.Cu) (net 14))
 (segment (start 80.01 119.7125) (end 78.74 120.9825) (width 0.25) (layer F.Cu) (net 14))
 (segment (start 80.01 114.3) (end 80.01 119.7125) (width 0.25) (layer F.Cu) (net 14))
 (segment (start 87.742 114.3) (end 80.01 114.3) (width 0.25) (layer F.Cu) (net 14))
 (segment (start 90.342 117.475) (end 90.342 116.9) (width 0.25) (layer F.Cu) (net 14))
 (segment (start 90.342 116.9) (end 87.742 114.3) (width 0.25) (layer F.Cu) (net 14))
 (segment (start 104.98 66.65) (end 110.53 72.2) (width 0.25) (layer F.Cu) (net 14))
 (segment (start 98.82 66.65) (end 104.98 66.65) (width 0.25) (layer F.Cu) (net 14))
 (segment (start 79.0725 123.19) (end 78.74 122.8575) (width 0.25) (layer F.Cu) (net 13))
 (segment (start 81.28 123.19) (end 79.0725 123.19) (width 0.25) (layer F.Cu) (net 13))
 (segment (start 78.4075 123.19) (end 78.74 122.8575) (width 0.25) (layer F.Cu) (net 13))
 (segment (start 75.102 123.19) (end 78.4075 123.19) (width 0.25) (layer F.Cu) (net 13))
 (segment (start 69.678 123.19) (end 75.102 123.19) (width 0.25) (layer F.Cu) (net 13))
 (segment (start 81.28 123.19) (end 81.28 115.57) (width 0.25) (layer F.Cu) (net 13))
 (segment (start 81.28 115.57) (end 87.63 115.57) (width 0.25) (layer F.Cu) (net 13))
 (segment (start 87.63 115.57) (end 87.63 119.38) (width 0.25) (layer F.Cu) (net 13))
 (segment (start 89.9045 121.285) (end 90.342 121.285) (width 0.25) (layer F.Cu) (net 13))
 (segment (start 87.9995 119.38) (end 89.9045 121.285) (width 0.25) (layer F.Cu) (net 13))
 (segment (start 87.63 119.38) (end 87.9995 119.38) (width 0.25) (layer F.Cu) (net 13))
 (segment (start 90.342 121.285) (end 90.342 122.092) (width 0.25) (layer F.Cu) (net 13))
 (segment (start 90.342 122.092) (end 91.44 123.19) (width 0.25) (layer F.Cu) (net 13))
 (segment (start 91.44 123.19) (end 91.44 123.19) (width 0.25) (layer F.Cu) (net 13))
 (via (at 91.44 123.19) (size 0.8) (drill 0.4) (layers F.Cu B.Cu) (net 13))
 (segment (start 86.6925 124.46) (end 85.09 124.46) (width 0.25) (layer F.Cu) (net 13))
 (segment (start 91.44 123.19) (end 85.09 123.19) (width 0.25) (layer B.Cu) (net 13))
 (via (at 85.09 123.19) (size 0.8) (drill 0.4) (layers F.Cu B.Cu) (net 13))
 (segment (start 85.09 124.46) (end 85.09 123.19) (width 0.25) (layer F.Cu) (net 13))
 (segment (start 107.95 120.65) (end 100.33 120.65) (width 0.25) (layer B.Cu) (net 13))
 (segment (start 97.79 123.19) (end 91.44 123.19) (width 0.25) (layer B.Cu) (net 13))
 (segment (start 100.33 120.65) (end 97.79 123.19) (width 0.25) (layer B.Cu) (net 13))
 (segment (start 107.95 112.49) (end 107.95 110.49) (width 0.25) (layer B.Cu) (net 13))
 (segment (start 107.41 113.03) (end 107.95 112.49) (width 0.25) (layer B.Cu) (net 13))
 (segment (start 102.87 113.03) (end 107.41 113.03) (width 0.25) (layer B.Cu) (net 13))
 (segment (start 107.95 120.65) (end 107.95 114.3) (width 0.25) (layer B.Cu) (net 13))
 (segment (start 107.41 113.76) (end 107.41 113.03) (width 0.25) (layer B.Cu) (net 13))
 (segment (start 107.95 114.3) (end 107.41 113.76) (width 0.25) (layer B.Cu) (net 13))
 (segment (start 107.95 108.49) (end 107.95 110.49) (width 0.25) (layer F.Cu) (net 13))
 (segment (start 113.57 102.87) (end 107.95 108.49) (width 0.25) (layer F.Cu) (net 13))
 (segment (start 118.11 102.87) (end 113.57 102.87) (width 0.25) (layer F.Cu) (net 13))
 (segment (start 119.38 101.6) (end 118.11 102.87) (width 0.25) (layer F.Cu) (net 13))
 (segment (start 120.65 101.6) (end 119.38 101.6) (width 0.25) (layer F.Cu) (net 13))
 (segment (start 94.22 71.29) (end 95.13 72.2) (width 0.25) (layer F.Cu) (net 13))
 (segment (start 94.22 66.65) (end 94.22 71.29) (width 0.25) (layer F.Cu) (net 13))
 (segment (start 75.102 124.46) (end 82.55 124.46) (width 0.25) (layer F.Cu) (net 19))
 (segment (start 82.55 123.795) (end 83.155 123.19) (width 0.25) (layer F.Cu) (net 19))
 (segment (start 82.55 124.46) (end 82.55 123.795) (width 0.25) (layer F.Cu) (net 19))
 (segment (start 84.918 121.427) (end 84.918 121.285) (width 0.25) (layer F.Cu) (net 19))
 (segment (start 83.155 123.19) (end 84.918 121.427) (width 0.25) (layer F.Cu) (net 19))
 (segment (start 82.55 126.395) (end 83.155 127) (width 0.25) (layer F.Cu) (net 19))
 (segment (start 82.55 124.46) (end 82.55 126.395) (width 0.25) (layer F.Cu) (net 19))
 (segment (start 100.33 101.6) (end 100.33 105.41) (width 0.25) (layer B.Cu) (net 26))
 (segment (start 119.38 105.41) (end 120.65 104.14) (width 0.25) (layer B.Cu) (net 26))
 (segment (start 100.33 105.41) (end 119.38 105.41) (width 0.25) (layer B.Cu) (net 26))
 (segment (start 109.14 97.79) (end 105.33 101.6) (width 0.25) (layer B.Cu) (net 27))
 (segment (start 120.65 99.06) (end 119.38 97.79) (width 0.25) (layer B.Cu) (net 27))
 (segment (start 119.38 97.79) (end 109.14 97.79) (width 0.25) (layer B.Cu) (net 27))
 (segment (start 90.7795 118.745) (end 90.342 118.745) (width 0.25) (layer F.Cu) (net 21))
 (segment (start 92.71 120.6755) (end 90.7795 118.745) (width 0.25) (layer F.Cu) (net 21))
 (segment (start 93.98 126.0625) (end 93.98 123.2155) (width 0.25) (layer F.Cu) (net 21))
 (segment (start 92.71 120.6755) (end 92.7355 120.6755) (width 0.25) (layer F.Cu) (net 21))
 (segment (start 92.7355 120.6755) (end 93.98 121.92) (width 0.25) (layer F.Cu) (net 21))
 (segment (start 93.98 121.92) (end 93.98 123.19) (width 0.25) (layer F.Cu) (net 21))
 (segment (start 84.918 117.475) (end 84.918 118.745) (width 0.25) (layer F.Cu) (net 22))
 (segment (start 91.1075 126.2) (end 91.1075 127) (width 0.25) (layer F.Cu) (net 22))
 (segment (start 91.1075 124.497) (end 91.1075 126.2) (width 0.25) (layer F.Cu) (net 22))
 (segment (start 85.3555 118.745) (end 91.1075 124.497) (width 0.25) (layer F.Cu) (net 22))
 (segment (start 84.918 118.745) (end 85.3555 118.745) (width 0.25) (layer F.Cu) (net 22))
 (segment (start 91.0705 124.46) (end 91.1075 124.497) (width 0.25) (layer F.Cu) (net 22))
 (segment (start 88.5675 124.46) (end 91.0705 124.46) (width 0.25) (layer F.Cu) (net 22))
 (segment (start 96.52 60.35) (end 96.52 66.65) (width 0.25) (layer F.Cu) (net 15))
 (segment (start 96.52 66.65) (end 96.52 69.85) (width 0.25) (layer F.Cu) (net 15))
 (segment (start 96.52 69.85) (end 99.06 72.39) (width 0.25) (layer F.Cu) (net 15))
 (segment (start 99.06 72.39) (end 99.06 74.93) (width 0.25) (layer F.Cu) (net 15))
 (segment (start 97.79 76.2) (end 46.99 76.2) (width 0.25) (layer F.Cu) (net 15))
 (segment (start 99.06 74.93) (end 97.79 76.2) (width 0.25) (layer F.Cu) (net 15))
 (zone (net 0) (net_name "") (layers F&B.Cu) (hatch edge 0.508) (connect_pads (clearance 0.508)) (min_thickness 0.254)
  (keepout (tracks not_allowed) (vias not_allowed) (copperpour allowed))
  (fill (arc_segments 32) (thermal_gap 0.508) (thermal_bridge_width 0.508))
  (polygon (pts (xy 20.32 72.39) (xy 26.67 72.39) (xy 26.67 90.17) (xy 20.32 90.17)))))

